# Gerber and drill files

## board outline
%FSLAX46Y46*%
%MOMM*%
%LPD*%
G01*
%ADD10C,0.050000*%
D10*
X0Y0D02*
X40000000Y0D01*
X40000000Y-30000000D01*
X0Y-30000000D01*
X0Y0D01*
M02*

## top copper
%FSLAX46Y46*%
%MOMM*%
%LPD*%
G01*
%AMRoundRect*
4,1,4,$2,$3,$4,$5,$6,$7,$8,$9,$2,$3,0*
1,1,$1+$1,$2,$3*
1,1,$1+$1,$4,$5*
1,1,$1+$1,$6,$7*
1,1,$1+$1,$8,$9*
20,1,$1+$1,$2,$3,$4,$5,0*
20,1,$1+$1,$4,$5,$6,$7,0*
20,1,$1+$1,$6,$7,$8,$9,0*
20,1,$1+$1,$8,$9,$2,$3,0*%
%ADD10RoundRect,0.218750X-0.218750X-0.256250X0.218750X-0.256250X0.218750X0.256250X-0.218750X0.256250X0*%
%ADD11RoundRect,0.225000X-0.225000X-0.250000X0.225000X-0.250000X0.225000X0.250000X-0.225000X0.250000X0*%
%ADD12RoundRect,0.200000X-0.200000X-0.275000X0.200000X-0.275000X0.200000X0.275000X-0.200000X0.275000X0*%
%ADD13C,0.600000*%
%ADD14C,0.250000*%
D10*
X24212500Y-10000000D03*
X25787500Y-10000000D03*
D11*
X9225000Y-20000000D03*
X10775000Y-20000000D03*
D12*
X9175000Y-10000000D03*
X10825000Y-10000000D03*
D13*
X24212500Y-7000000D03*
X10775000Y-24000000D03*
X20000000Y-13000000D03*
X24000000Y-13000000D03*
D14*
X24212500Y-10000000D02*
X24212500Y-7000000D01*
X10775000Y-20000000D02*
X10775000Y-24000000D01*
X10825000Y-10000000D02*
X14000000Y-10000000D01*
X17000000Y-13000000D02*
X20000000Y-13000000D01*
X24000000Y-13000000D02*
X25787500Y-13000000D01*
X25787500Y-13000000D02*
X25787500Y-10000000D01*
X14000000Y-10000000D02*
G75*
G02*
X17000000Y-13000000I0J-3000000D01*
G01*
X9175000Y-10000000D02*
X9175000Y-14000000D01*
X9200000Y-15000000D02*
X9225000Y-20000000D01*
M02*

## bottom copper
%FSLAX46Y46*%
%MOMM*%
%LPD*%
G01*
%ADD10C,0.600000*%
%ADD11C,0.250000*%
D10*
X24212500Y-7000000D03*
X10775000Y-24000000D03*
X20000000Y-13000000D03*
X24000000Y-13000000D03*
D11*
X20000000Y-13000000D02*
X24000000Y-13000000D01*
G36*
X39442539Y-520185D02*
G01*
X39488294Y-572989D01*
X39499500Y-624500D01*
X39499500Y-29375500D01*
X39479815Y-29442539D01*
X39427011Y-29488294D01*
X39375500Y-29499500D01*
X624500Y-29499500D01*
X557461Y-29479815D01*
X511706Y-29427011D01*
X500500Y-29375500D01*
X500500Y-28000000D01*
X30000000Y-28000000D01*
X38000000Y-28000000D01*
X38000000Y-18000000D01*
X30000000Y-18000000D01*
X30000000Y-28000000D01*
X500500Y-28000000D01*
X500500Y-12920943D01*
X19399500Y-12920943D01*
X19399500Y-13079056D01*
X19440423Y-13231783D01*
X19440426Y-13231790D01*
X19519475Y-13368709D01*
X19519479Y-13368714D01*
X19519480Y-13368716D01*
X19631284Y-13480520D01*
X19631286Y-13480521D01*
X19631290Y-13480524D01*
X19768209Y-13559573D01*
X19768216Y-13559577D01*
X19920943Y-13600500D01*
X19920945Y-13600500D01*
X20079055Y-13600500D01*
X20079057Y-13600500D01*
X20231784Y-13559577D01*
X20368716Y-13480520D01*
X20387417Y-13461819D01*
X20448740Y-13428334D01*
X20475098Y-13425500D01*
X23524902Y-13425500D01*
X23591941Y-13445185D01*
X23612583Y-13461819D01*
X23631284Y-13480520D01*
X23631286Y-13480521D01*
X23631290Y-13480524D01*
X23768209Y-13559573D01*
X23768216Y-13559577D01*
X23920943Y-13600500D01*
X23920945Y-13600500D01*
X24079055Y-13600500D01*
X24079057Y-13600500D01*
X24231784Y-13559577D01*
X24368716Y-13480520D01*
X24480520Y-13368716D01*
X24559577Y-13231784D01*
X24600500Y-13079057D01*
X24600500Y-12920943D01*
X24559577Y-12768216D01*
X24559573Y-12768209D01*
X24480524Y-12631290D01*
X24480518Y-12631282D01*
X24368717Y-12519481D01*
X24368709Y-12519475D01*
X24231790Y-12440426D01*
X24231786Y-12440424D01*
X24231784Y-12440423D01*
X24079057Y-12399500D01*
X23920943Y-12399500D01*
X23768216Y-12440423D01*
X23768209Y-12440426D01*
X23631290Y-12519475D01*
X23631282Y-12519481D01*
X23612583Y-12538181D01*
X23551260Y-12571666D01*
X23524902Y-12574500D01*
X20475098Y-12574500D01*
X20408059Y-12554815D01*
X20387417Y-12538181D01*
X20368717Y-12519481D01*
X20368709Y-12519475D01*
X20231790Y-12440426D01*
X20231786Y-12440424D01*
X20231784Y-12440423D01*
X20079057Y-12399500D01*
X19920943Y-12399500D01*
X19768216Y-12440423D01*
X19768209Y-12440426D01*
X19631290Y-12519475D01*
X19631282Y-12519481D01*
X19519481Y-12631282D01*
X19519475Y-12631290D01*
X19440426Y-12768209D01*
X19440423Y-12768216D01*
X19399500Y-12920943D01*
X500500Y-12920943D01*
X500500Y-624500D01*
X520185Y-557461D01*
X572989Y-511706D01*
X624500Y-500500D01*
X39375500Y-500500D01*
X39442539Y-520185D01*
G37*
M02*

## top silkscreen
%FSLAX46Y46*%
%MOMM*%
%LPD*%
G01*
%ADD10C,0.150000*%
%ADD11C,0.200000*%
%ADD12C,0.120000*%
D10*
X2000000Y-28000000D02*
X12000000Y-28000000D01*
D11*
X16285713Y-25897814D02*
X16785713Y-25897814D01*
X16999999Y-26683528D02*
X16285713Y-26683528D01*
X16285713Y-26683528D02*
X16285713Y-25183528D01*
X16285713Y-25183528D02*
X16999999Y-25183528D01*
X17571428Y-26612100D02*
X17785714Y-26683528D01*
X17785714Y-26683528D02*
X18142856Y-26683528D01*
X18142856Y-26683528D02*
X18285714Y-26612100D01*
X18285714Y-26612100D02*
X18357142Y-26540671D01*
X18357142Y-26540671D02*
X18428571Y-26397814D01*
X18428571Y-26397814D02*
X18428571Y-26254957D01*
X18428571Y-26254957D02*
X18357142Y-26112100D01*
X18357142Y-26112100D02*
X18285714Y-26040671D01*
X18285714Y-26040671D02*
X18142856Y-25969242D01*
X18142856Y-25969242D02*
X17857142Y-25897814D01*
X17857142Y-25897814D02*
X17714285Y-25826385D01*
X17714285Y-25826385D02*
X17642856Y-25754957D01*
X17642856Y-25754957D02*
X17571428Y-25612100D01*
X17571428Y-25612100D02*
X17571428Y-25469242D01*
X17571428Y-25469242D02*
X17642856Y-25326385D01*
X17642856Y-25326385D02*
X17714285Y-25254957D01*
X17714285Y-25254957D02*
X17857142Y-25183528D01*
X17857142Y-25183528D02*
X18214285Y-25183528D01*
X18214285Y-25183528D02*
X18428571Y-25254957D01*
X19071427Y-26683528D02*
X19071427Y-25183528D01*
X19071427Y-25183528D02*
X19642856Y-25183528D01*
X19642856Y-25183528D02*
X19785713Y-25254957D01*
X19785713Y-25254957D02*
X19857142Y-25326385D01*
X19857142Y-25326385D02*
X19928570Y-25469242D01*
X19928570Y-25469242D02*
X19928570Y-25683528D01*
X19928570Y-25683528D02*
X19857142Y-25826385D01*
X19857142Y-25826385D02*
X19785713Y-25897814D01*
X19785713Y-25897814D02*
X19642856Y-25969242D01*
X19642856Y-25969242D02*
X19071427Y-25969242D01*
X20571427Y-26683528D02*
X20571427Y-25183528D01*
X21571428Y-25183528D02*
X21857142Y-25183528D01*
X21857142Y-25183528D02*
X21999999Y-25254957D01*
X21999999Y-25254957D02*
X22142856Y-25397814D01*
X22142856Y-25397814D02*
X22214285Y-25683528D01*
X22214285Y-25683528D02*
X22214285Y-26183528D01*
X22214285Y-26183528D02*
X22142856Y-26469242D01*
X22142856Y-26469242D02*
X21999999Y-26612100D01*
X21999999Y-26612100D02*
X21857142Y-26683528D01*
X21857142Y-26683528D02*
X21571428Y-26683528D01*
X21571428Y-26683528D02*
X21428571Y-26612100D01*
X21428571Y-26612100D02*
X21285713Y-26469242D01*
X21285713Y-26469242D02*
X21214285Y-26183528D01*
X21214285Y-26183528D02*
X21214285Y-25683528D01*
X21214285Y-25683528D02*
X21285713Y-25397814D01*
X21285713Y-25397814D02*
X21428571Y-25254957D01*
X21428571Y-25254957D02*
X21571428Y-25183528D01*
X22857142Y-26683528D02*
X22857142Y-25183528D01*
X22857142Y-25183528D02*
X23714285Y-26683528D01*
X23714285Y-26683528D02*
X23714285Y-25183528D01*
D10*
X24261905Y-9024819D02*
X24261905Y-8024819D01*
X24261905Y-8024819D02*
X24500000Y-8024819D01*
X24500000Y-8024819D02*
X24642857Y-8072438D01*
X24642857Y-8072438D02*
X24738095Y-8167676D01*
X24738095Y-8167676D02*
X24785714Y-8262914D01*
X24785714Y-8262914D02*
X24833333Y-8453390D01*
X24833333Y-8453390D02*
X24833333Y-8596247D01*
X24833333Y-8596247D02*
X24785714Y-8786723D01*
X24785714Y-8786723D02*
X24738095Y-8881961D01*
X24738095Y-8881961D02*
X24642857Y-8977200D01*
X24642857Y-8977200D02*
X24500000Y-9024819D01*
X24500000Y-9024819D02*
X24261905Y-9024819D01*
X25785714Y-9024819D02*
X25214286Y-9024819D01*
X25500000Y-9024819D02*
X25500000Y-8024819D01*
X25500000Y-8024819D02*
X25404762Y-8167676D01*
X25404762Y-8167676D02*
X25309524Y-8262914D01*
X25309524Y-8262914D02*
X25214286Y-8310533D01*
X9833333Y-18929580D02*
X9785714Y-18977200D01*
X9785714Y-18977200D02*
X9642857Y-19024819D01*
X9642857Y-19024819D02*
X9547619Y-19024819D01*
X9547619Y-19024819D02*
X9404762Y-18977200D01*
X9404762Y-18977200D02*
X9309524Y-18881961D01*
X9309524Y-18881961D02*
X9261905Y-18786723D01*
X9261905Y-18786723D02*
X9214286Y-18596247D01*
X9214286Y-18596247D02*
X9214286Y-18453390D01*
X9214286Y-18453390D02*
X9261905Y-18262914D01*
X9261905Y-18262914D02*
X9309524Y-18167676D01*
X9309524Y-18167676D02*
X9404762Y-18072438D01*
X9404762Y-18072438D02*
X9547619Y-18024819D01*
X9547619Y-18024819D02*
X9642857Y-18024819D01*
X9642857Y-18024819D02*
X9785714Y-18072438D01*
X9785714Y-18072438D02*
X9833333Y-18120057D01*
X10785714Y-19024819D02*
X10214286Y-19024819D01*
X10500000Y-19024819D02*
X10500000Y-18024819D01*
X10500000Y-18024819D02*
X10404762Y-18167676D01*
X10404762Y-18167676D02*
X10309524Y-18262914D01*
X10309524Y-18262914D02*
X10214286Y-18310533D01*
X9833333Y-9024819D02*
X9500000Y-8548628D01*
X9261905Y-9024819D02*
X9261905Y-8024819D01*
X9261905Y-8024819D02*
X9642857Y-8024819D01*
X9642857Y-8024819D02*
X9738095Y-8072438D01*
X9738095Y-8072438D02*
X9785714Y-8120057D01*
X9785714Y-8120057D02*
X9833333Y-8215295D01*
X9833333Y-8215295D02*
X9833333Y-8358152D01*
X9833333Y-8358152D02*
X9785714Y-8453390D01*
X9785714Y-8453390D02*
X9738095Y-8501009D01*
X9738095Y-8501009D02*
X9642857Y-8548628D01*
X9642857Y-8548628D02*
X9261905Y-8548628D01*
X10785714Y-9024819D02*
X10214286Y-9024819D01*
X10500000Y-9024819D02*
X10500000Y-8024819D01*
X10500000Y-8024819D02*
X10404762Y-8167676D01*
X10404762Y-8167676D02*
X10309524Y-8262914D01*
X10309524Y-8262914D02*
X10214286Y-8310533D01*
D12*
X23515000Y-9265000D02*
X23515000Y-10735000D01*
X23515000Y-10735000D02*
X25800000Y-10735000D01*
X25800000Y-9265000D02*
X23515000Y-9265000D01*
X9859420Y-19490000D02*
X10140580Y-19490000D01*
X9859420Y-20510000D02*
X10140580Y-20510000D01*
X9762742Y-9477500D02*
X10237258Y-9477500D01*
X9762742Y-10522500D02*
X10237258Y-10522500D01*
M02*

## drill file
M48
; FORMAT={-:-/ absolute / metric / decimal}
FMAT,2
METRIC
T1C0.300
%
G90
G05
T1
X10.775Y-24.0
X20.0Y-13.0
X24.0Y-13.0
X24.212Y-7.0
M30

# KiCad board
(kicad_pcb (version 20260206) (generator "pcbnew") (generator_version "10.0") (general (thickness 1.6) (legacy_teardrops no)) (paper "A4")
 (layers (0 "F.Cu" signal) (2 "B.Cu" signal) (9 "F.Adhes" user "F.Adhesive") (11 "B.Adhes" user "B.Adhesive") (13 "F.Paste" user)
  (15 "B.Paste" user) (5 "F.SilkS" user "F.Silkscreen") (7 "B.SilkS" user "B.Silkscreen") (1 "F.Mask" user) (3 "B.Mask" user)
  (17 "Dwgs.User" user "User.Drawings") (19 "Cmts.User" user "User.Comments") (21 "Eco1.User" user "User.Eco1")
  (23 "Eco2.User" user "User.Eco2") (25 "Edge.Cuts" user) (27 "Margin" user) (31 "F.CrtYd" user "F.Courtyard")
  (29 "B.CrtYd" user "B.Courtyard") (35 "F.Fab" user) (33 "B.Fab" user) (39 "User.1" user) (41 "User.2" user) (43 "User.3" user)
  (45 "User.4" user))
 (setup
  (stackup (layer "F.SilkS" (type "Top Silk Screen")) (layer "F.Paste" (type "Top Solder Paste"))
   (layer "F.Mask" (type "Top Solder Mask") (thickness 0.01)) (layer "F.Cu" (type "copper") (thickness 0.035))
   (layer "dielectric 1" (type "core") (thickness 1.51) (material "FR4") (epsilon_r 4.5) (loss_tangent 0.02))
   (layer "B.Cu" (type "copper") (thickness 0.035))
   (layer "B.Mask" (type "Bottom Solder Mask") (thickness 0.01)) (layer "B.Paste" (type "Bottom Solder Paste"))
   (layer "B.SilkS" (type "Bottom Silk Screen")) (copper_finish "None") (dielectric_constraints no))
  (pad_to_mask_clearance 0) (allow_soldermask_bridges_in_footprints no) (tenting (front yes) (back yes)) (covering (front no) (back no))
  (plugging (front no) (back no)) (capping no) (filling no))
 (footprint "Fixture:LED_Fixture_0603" (layer "F.Cu") (at 25 10)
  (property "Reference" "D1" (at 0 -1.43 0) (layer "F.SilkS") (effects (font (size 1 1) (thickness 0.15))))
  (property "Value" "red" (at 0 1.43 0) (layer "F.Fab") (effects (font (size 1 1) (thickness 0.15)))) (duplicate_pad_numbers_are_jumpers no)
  (fp_line (start -1.485 -0.735) (end -1.485 0.735) (stroke (width 0.12) (type solid)) (layer "F.SilkS"))
  (fp_line (start -1.485 0.735) (end 0.8 0.735) (stroke (width 0.12) (type solid)) (layer "F.SilkS"))
  (fp_line (start 0.8 -0.735) (end -1.485 -0.735) (stroke (width 0.12) (type solid)) (layer "F.SilkS"))
  (pad "1" smd roundrect (at -0.7875 0) (size 0.875 0.95) (layers "F.Cu" "F.Mask" "F.Paste") (roundrect_rratio 0.25) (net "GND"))
  (pad "2" smd roundrect (at 0.7875 0) (size 0.875 0.95) (layers "F.Cu" "F.Mask" "F.Paste") (roundrect_rratio 0.25) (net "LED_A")))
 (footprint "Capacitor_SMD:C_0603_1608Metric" (layer "F.Cu") (at 10 20)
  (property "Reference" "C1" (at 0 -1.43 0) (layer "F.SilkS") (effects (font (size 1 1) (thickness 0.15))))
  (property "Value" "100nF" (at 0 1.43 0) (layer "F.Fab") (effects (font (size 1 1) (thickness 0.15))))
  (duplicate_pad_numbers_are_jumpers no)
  (fp_line (start -0.14058 -0.51) (end 0.14058 -0.51) (stroke (width 0.12) (type solid)) (layer "F.SilkS"))
  (fp_line (start -0.14058 0.51) (end 0.14058 0.51) (stroke (width 0.12) (type solid)) (layer "F.SilkS"))
  (pad "1" smd roundrect (at -0.775 0) (size 0.9 0.95) (layers "F.Cu" "F.Mask" "F.Paste") (roundrect_rratio 0.25) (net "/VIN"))
  (pad "2" smd roundrect (at 0.775 0) (size 0.9 0.95) (layers "F.Cu" "F.Mask" "F.Paste") (roundrect_rratio 0.25) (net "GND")))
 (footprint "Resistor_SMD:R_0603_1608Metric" (layer "F.Cu") (at 10 10)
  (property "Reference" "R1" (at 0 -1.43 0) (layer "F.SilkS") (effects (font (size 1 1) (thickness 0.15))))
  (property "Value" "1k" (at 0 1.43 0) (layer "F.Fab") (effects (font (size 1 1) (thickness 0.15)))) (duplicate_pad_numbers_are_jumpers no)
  (fp_line (start -0.237258 -0.5225) (end 0.237258 -0.5225) (stroke (width 0.12) (type solid)) (layer "F.SilkS"))
  (fp_line (start -0.237258 0.5225) (end 0.237258 0.5225) (stroke (width 0.12) (type solid)) (layer "F.SilkS"))
  (pad "1" smd roundrect (at -0.825 0) (size 0.8 0.95) (layers "F.Cu" "F.Mask" "F.Paste") (roundrect_rratio 0.25) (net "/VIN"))
  (pad "2" smd roundrect (at 0.825 0) (size 0.8 0.95) (layers "F.Cu" "F.Mask" "F.Paste") (roundrect_rratio 0.25) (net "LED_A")))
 (gr_line (start 2 28) (end 12 28) (stroke (width 0.15) (type solid)) (layer "F.SilkS"))
 (gr_rect (start 0 0) (end 40 30) (stroke (width 0.05) (type default)) (fill no) (layer "Edge.Cuts"))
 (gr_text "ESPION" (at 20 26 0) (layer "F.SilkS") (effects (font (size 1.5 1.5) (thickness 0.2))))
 (segment (start 24.2125 10) (end 24.2125 7) (width 0.25) (layer "F.Cu") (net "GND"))
 (segment (start 10.775 20) (end 10.775 24) (width 0.25) (layer "F.Cu") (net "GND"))
 (via (at 24.2125 7) (size 0.6) (drill 0.3) (layers "F.Cu" "B.Cu") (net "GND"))
 (via (at 10.775 24) (size 0.6) (drill 0.3) (layers "F.Cu" "B.Cu") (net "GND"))
 (segment (start 10.825 10) (end 14 10) (width 0.25) (layer "F.Cu") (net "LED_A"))
 (segment (start 17 13) (end 20 13) (width 0.25) (layer "F.Cu") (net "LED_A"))
 (segment (start 24 13) (end 25.7875 13) (width 0.25) (layer "F.Cu") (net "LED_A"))
 (segment (start 25.7875 13) (end 25.7875 10) (width 0.25) (layer "F.Cu") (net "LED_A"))
 (via (at 20 13) (size 0.6) (drill 0.3) (layers "F.Cu" "B.Cu") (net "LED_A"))
 (via (at 24 13) (size 0.6) (drill 0.3) (layers "F.Cu" "B.Cu") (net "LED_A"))
 (arc (start 14 10) (mid 16.12132 10.87868) (end 17 13) (width 0.25) (layer "F.Cu") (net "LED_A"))
 (segment (start 20 13) (end 24 13) (width 0.25) (layer "B.Cu") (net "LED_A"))
 (segment (start 9.175 10) (end 9.175 14) (width 0.25) (layer "F.Cu") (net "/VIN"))
 (segment (start 9.2 15) (end 9.225 20) (width 0.25) (layer "F.Cu") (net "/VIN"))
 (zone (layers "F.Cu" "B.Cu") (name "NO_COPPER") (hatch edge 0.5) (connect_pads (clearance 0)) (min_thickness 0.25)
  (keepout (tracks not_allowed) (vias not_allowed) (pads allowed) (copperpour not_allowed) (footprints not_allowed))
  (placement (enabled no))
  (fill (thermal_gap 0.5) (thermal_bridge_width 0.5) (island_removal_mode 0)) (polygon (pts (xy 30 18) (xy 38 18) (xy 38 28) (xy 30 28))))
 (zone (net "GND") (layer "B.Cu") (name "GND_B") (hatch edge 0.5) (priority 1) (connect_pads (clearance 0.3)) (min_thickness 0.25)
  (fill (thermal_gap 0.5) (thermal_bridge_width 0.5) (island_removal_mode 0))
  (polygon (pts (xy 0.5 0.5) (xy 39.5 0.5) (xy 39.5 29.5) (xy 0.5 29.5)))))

